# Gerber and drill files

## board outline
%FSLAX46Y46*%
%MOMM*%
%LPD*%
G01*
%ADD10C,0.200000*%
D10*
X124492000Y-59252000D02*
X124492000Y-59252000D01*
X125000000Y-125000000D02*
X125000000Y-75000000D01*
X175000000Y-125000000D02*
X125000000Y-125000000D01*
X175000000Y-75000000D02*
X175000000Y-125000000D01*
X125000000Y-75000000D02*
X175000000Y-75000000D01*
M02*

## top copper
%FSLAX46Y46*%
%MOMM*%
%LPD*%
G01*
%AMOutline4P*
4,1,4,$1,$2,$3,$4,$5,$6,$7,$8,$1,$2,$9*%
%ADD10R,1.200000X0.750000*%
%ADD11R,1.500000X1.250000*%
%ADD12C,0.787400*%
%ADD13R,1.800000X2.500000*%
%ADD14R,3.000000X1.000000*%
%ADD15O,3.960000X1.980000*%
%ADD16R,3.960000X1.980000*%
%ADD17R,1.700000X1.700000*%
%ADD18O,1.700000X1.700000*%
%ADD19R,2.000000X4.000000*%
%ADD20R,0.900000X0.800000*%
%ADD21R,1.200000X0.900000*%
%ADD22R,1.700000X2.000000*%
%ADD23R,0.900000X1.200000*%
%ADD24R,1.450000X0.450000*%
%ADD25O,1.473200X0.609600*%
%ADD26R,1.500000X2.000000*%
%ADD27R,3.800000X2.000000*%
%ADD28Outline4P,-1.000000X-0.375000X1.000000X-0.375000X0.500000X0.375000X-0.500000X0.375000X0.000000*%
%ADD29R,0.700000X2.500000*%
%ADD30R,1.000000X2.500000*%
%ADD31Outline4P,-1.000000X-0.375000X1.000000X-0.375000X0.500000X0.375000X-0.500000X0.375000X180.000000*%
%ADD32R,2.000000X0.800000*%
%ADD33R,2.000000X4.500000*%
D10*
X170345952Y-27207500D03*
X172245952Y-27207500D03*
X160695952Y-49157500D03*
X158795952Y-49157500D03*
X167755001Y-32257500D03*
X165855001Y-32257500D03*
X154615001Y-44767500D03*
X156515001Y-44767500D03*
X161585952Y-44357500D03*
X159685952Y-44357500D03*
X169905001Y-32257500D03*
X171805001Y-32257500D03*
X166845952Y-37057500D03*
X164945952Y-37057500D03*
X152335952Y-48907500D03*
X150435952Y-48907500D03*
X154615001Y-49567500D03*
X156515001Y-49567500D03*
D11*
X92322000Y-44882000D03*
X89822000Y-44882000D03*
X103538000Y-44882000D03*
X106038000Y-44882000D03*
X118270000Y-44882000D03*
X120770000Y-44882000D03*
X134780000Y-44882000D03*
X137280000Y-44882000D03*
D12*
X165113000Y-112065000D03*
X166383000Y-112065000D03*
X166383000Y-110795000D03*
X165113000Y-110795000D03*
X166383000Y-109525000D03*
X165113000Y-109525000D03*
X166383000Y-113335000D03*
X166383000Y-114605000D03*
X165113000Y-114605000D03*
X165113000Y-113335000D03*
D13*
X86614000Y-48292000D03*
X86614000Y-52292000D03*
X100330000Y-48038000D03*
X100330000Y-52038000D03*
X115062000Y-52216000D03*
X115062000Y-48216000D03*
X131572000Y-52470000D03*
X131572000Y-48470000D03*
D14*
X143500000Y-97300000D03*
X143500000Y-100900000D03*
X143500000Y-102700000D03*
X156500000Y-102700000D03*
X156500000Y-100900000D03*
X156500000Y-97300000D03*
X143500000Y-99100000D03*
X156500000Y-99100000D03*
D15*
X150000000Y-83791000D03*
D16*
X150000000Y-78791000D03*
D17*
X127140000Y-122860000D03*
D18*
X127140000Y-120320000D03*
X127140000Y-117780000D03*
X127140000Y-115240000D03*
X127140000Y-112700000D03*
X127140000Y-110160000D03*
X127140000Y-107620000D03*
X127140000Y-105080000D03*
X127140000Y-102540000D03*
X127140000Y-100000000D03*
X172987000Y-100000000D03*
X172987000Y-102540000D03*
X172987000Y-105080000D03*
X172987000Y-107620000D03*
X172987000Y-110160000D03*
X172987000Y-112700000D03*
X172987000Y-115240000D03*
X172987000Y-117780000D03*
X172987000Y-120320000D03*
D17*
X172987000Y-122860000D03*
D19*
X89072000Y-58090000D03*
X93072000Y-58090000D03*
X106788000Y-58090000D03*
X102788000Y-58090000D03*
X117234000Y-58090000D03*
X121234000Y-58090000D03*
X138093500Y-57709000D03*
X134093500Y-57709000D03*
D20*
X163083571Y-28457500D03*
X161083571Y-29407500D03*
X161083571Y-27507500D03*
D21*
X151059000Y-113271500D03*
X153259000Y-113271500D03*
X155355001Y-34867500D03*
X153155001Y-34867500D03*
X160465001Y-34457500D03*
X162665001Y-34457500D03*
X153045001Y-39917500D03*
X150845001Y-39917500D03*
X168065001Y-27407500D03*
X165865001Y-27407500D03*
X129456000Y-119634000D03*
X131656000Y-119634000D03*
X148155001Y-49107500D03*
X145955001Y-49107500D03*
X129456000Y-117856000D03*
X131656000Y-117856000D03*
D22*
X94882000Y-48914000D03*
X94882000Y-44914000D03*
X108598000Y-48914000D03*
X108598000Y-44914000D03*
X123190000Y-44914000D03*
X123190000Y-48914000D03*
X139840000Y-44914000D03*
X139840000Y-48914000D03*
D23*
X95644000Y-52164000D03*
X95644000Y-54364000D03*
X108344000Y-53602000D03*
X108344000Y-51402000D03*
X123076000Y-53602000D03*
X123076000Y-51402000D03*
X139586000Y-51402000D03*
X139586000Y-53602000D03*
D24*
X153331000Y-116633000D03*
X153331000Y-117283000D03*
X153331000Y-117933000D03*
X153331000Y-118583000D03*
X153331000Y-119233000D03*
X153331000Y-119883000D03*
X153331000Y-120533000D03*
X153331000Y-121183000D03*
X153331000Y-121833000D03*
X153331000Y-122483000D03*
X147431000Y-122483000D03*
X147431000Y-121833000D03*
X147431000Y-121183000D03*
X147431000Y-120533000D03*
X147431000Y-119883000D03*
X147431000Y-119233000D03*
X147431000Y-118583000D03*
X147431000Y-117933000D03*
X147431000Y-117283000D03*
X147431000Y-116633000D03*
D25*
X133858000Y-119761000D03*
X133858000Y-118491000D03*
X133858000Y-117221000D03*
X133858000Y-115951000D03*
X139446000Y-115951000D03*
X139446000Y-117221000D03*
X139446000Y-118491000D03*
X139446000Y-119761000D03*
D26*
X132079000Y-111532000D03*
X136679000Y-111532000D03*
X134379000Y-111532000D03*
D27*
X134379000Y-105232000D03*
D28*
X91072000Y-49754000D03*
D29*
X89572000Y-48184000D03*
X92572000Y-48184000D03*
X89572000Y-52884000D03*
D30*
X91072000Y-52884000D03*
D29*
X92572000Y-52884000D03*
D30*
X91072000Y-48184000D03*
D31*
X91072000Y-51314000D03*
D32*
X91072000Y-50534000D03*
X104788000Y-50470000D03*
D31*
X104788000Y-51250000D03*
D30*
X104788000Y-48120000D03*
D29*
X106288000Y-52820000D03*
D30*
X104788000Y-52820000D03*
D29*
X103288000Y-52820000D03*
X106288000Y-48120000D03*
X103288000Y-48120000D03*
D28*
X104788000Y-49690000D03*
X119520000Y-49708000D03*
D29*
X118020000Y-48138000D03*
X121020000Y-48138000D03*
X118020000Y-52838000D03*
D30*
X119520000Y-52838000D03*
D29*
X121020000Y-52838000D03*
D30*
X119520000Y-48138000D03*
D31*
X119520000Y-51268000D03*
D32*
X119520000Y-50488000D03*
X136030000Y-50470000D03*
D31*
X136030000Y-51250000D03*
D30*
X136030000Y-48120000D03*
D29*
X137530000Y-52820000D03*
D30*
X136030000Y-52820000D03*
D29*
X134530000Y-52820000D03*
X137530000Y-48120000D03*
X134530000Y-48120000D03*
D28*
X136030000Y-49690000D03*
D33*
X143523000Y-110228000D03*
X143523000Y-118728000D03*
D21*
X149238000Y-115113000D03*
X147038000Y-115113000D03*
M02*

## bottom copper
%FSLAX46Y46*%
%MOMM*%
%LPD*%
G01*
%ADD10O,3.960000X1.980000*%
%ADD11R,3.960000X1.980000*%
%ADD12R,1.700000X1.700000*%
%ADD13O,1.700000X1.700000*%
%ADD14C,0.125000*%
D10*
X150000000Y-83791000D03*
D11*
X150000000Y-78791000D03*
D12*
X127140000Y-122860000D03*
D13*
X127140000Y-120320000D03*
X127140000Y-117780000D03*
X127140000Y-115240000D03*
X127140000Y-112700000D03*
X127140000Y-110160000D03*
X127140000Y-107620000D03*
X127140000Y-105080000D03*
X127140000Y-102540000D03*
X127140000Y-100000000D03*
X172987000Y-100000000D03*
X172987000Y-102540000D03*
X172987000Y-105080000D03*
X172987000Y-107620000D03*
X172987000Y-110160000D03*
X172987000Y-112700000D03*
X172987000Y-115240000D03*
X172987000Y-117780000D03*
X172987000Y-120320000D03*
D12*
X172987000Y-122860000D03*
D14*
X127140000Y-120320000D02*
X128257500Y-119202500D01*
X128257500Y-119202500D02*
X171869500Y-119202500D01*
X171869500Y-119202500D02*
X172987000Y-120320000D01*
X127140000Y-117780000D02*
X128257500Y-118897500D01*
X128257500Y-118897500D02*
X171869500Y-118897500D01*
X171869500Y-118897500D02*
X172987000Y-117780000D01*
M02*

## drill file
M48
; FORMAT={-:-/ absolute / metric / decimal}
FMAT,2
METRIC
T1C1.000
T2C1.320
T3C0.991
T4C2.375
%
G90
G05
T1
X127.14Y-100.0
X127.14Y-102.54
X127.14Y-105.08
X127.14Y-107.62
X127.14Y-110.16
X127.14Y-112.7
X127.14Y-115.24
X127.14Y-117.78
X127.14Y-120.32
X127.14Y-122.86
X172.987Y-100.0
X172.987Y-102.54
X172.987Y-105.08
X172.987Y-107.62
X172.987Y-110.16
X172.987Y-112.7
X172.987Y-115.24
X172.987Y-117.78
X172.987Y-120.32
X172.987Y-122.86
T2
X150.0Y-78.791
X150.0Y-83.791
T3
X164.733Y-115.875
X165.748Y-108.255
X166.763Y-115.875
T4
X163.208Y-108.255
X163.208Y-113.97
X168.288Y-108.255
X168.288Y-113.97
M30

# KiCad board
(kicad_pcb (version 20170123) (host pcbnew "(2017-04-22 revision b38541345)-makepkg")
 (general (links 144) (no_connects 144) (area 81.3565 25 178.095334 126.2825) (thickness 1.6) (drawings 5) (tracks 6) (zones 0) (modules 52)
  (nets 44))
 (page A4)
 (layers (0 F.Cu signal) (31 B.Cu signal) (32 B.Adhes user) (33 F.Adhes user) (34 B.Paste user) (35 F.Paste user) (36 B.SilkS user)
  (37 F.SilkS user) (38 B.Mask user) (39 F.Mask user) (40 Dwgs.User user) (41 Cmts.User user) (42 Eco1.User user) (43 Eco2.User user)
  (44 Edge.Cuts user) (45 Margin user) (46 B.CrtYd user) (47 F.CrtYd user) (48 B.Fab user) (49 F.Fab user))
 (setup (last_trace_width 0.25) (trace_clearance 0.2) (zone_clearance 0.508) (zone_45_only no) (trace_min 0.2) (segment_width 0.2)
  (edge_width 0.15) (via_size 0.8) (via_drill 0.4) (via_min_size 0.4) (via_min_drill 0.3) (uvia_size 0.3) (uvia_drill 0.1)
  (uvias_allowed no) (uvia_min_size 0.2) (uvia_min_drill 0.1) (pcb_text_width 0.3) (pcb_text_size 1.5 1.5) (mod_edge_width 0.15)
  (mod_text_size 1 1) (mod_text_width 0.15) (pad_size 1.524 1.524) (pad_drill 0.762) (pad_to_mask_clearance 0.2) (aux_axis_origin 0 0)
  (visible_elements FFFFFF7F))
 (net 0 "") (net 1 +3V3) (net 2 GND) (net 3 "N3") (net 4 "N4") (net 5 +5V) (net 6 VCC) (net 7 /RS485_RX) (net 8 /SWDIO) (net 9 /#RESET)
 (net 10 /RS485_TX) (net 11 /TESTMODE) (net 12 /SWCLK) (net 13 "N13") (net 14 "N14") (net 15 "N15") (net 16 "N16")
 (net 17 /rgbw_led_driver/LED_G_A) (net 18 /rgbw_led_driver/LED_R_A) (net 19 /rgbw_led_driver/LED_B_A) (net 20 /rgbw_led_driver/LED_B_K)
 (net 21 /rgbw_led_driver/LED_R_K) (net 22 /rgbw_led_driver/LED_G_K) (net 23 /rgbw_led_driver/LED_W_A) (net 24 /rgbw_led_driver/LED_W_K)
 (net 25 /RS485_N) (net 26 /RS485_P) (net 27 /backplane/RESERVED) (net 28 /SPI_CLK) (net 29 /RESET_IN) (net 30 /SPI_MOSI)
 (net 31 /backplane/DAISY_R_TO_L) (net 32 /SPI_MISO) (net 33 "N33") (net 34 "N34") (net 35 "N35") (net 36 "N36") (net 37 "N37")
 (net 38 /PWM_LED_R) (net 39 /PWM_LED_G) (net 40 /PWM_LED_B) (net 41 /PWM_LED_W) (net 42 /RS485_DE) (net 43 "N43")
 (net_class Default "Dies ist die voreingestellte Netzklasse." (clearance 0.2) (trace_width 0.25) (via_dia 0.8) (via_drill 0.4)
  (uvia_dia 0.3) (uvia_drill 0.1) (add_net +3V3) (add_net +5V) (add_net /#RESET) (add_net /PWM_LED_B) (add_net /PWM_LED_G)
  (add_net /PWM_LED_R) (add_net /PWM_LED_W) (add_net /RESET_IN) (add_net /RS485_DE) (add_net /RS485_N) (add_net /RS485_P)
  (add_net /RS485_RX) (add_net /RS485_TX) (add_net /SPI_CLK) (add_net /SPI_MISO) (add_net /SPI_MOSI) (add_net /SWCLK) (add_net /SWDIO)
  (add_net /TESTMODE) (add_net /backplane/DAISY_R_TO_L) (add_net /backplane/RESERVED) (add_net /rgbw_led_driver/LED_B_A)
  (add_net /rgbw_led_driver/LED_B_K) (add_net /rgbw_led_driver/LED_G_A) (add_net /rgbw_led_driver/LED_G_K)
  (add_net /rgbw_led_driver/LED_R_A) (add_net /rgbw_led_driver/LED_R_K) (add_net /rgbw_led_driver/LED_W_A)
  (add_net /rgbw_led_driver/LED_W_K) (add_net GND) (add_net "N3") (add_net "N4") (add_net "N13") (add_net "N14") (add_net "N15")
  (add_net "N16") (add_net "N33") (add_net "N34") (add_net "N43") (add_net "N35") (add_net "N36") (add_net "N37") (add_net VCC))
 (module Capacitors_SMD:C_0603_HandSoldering (layer F.Cu) (at 171.295952 27.2075)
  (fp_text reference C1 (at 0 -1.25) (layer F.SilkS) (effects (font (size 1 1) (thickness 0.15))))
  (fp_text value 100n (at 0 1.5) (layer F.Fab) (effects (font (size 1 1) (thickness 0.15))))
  (pad 1 smd rect (at -0.95 0) (size 1.2 0.75) (layers F.Cu F.Paste F.Mask) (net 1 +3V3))
  (pad 2 smd rect (at 0.95 0) (size 1.2 0.75) (layers F.Cu F.Paste F.Mask) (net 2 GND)))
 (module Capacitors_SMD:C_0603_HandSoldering (layer F.Cu) (at 159.745952 49.1575)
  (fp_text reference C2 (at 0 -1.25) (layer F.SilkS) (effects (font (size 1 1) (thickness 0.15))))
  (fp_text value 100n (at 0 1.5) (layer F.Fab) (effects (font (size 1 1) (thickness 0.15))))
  (pad 2 smd rect (at 0.95 0) (size 1.2 0.75) (layers F.Cu F.Paste F.Mask) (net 2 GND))
  (pad 1 smd rect (at -0.95 0) (size 1.2 0.75) (layers F.Cu F.Paste F.Mask) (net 1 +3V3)))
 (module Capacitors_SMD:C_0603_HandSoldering (layer F.Cu) (at 166.805001 32.2575)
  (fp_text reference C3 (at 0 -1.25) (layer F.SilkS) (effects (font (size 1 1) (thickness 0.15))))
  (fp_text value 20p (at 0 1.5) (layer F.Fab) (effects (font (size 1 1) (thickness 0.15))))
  (pad 2 smd rect (at 0.95 0) (size 1.2 0.75) (layers F.Cu F.Paste F.Mask) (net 2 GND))
  (pad 1 smd rect (at -0.95 0) (size 1.2 0.75) (layers F.Cu F.Paste F.Mask) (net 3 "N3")))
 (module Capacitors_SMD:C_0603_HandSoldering (layer F.Cu) (at 155.565001 44.7675)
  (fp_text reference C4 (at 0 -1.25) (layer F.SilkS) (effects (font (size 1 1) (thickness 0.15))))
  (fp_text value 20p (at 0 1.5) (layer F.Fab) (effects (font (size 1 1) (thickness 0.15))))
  (pad 1 smd rect (at -0.95 0) (size 1.2 0.75) (layers F.Cu F.Paste F.Mask) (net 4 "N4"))
  (pad 2 smd rect (at 0.95 0) (size 1.2 0.75) (layers F.Cu F.Paste F.Mask) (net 2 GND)))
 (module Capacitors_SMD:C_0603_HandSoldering (layer F.Cu) (at 160.635952 44.3575)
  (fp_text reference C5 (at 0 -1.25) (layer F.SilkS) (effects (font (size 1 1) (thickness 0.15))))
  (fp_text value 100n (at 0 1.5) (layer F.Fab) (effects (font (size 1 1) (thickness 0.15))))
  (pad 2 smd rect (at 0.95 0) (size 1.2 0.75) (layers F.Cu F.Paste F.Mask) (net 2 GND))
  (pad 1 smd rect (at -0.95 0) (size 1.2 0.75) (layers F.Cu F.Paste F.Mask) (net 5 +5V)))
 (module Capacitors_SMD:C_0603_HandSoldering (layer F.Cu) (at 170.855001 32.2575)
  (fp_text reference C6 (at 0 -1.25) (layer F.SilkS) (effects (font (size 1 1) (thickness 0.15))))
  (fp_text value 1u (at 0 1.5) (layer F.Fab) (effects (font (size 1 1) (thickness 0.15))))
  (pad 1 smd rect (at -0.95 0) (size 1.2 0.75) (layers F.Cu F.Paste F.Mask) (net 5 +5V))
  (pad 2 smd rect (at 0.95 0) (size 1.2 0.75) (layers F.Cu F.Paste F.Mask) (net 2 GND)))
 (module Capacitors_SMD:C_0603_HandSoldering (layer F.Cu) (at 165.895952 37.0575)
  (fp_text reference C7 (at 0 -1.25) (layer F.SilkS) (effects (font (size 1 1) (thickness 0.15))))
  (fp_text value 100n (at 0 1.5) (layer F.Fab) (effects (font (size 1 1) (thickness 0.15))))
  (pad 2 smd rect (at 0.95 0) (size 1.2 0.75) (layers F.Cu F.Paste F.Mask) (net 2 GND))
  (pad 1 smd rect (at -0.95 0) (size 1.2 0.75) (layers F.Cu F.Paste F.Mask) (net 5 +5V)))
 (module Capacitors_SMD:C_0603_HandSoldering (layer F.Cu) (at 151.385952 48.9075)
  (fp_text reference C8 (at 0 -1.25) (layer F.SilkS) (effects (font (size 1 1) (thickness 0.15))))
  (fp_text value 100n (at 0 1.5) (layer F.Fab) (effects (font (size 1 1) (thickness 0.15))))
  (pad 2 smd rect (at 0.95 0) (size 1.2 0.75) (layers F.Cu F.Paste F.Mask) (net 2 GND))
  (pad 1 smd rect (at -0.95 0) (size 1.2 0.75) (layers F.Cu F.Paste F.Mask) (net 1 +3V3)))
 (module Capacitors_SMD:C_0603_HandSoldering (layer F.Cu) (at 155.565001 49.5675)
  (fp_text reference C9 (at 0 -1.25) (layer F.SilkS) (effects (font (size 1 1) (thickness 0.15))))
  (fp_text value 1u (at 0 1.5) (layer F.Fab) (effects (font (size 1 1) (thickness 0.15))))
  (pad 1 smd rect (at -0.95 0) (size 1.2 0.75) (layers F.Cu F.Paste F.Mask) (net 1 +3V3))
  (pad 2 smd rect (at 0.95 0) (size 1.2 0.75) (layers F.Cu F.Paste F.Mask) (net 2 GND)))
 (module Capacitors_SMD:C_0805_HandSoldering (layer F.Cu) (at 91.072 44.882)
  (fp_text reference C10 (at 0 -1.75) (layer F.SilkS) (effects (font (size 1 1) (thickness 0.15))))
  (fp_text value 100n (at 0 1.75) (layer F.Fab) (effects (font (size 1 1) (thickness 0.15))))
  (pad 2 smd rect (at 1.25 0) (size 1.5 1.25) (layers F.Cu F.Paste F.Mask) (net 2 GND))
  (pad 1 smd rect (at -1.25 0) (size 1.5 1.25) (layers F.Cu F.Paste F.Mask) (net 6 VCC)))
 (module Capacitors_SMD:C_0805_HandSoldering (layer F.Cu) (at 104.788 44.882)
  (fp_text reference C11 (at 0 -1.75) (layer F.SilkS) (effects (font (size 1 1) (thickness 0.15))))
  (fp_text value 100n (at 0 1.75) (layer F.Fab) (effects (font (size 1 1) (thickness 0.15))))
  (pad 1 smd rect (at -1.25 0) (size 1.5 1.25) (layers F.Cu F.Paste F.Mask) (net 6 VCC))
  (pad 2 smd rect (at 1.25 0) (size 1.5 1.25) (layers F.Cu F.Paste F.Mask) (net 2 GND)))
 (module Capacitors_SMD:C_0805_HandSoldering (layer F.Cu) (at 119.52 44.882)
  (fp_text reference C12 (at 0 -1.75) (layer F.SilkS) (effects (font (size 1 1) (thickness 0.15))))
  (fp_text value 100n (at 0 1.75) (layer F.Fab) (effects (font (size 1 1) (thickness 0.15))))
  (pad 1 smd rect (at -1.25 0) (size 1.5 1.25) (layers F.Cu F.Paste F.Mask) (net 6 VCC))
  (pad 2 smd rect (at 1.25 0) (size 1.5 1.25) (layers F.Cu F.Paste F.Mask) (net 2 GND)))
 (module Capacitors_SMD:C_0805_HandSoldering (layer F.Cu) (at 136.03 44.882)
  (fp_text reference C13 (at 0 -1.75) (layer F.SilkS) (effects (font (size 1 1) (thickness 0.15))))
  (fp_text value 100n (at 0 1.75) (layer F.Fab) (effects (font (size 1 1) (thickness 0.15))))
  (pad 1 smd rect (at -1.25 0) (size 1.5 1.25) (layers F.Cu F.Paste F.Mask) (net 6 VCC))
  (pad 2 smd rect (at 1.25 0) (size 1.5 1.25) (layers F.Cu F.Paste F.Mask) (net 2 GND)))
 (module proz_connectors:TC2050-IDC (layer F.Cu) (at 165.748 112.065 270)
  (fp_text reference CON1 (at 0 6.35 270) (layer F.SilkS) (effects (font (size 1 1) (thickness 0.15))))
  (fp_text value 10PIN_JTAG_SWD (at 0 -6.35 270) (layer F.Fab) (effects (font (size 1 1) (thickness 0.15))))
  (pad 3 smd circle (at 0 0.635 270) (size 0.7874 0.7874) (layers F.Cu F.Mask) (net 2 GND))
  (pad 8 smd circle (at 0 -0.635 270) (size 0.7874 0.7874) (layers F.Cu F.Mask))
  (pad 9 smd circle (at -1.27 -0.635 270) (size 0.7874 0.7874) (layers F.Cu F.Mask) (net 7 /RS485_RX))
  (pad 2 smd circle (at -1.27 0.635 270) (size 0.7874 0.7874) (layers F.Cu F.Mask) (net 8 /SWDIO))
  (pad 10 smd circle (at -2.54 -0.635 270) (size 0.7874 0.7874) (layers F.Cu F.Mask) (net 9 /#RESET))
  (pad 1 smd circle (at -2.54 0.635 270) (size 0.7874 0.7874) (layers F.Cu F.Mask) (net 1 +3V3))
  (pad 7 smd circle (at 1.27 -0.635 270) (size 0.7874 0.7874) (layers F.Cu F.Mask) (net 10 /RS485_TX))
  (pad 6 smd circle (at 2.54 -0.635 270) (size 0.7874 0.7874) (layers F.Cu F.Mask))
  (pad 5 smd circle (at 2.54 0.635 270) (size 0.7874 0.7874) (layers F.Cu F.Mask) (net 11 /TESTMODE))
  (pad 4 smd circle (at 1.27 0.635 270) (size 0.7874 0.7874) (layers F.Cu F.Mask) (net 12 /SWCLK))
  (pad "" np_thru_hole circle (at -3.81 -2.54 270) (size 2.375 2.375) (drill 2.375) (layers *.Cu *.Mask F.SilkS))
  (pad "" np_thru_hole circle (at -3.81 0 270) (size 0.9906 0.9906) (drill 0.9906) (layers *.Cu *.Mask F.SilkS))
  (pad "" np_thru_hole circle (at 3.81 -1.015 270) (size 0.9906 0.9906) (drill 0.9906) (layers *.Cu *.Mask F.SilkS))
  (pad "" np_thru_hole circle (at 3.81 1.015 270) (size 0.9906 0.9906) (drill 0.9906) (layers *.Cu *.Mask F.SilkS))
  (pad "" np_thru_hole circle (at -3.81 2.54 270) (size 2.375 2.375) (drill 2.375) (layers *.Cu *.Mask F.SilkS))
  (pad "" np_thru_hole circle (at 1.905 2.54 270) (size 2.375 2.375) (drill 2.375) (layers *.Cu *.Mask F.SilkS))
  (pad "" np_thru_hole circle (at 1.905 -2.54 270) (size 2.375 2.375) (drill 2.375) (layers *.Cu *.Mask F.SilkS)))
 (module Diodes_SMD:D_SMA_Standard (layer F.Cu) (at 86.614 50.292 270)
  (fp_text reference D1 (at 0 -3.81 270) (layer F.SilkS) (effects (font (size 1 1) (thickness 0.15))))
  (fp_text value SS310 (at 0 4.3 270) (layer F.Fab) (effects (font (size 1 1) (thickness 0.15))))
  (pad 1 smd rect (at -2 0 270) (size 2.5 1.8) (layers F.Cu F.Paste F.Mask) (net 6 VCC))
  (pad 2 smd rect (at 2 0 270) (size 2.5 1.8) (layers F.Cu F.Paste F.Mask) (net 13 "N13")))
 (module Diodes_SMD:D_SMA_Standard (layer F.Cu) (at 100.33 50.038 270)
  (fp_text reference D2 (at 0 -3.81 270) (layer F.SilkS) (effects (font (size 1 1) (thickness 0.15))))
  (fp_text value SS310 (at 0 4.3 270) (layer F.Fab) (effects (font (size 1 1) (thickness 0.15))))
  (pad 1 smd rect (at -2 0 270) (size 2.5 1.8) (layers F.Cu F.Paste F.Mask) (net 6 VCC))
  (pad 2 smd rect (at 2 0 270) (size 2.5 1.8) (layers F.Cu F.Paste F.Mask) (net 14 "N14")))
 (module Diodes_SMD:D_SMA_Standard (layer F.Cu) (at 115.062 50.216 270)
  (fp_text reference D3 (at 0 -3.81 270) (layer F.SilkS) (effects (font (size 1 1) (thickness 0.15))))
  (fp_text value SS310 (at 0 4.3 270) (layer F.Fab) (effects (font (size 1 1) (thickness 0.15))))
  (pad 2 smd rect (at 2 0 270) (size 2.5 1.8) (layers F.Cu F.Paste F.Mask) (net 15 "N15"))
  (pad 1 smd rect (at -2 0 270) (size 2.5 1.8) (layers F.Cu F.Paste F.Mask) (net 6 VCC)))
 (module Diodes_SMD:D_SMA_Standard (layer F.Cu) (at 131.572 50.47 270)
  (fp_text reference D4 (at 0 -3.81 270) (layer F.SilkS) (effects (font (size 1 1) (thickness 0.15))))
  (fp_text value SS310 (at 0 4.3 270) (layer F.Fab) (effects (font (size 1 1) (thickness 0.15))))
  (pad 2 smd rect (at 2 0 270) (size 2.5 1.8) (layers F.Cu F.Paste F.Mask) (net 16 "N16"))
  (pad 1 smd rect (at -2 0 270) (size 2.5 1.8) (layers F.Cu F.Paste F.Mask) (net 6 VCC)))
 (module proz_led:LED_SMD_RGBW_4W (layer F.Cu) (at 150 100)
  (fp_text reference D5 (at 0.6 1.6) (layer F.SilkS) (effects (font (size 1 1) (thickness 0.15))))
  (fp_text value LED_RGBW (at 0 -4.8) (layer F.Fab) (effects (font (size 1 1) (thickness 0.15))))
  (pad 8 smd rect (at -6.5 -2.7) (size 3 1) (layers F.Cu F.Paste F.Mask) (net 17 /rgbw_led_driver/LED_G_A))
  (pad 6 smd rect (at -6.5 0.9) (size 3 1) (layers F.Cu F.Paste F.Mask) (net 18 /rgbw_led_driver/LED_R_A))
  (pad 5 smd rect (at -6.5 2.7) (size 3 1) (layers F.Cu F.Paste F.Mask) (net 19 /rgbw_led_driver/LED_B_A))
  (pad 4 smd rect (at 6.5 2.7) (size 3 1) (layers F.Cu F.Paste F.Mask) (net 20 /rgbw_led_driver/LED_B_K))
  (pad 3 smd rect (at 6.5 0.9) (size 3 1) (layers F.Cu F.Paste F.Mask) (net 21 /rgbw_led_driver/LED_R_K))
  (pad 1 smd rect (at 6.5 -2.7) (size 3 1) (layers F.Cu F.Paste F.Mask) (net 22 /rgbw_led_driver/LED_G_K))
  (pad "" smd circle (at 0 0) (size 7.5 7.5) (layers F.Mask))
  (pad 7 smd rect (at -6.5 -0.9) (size 3 1) (layers F.Cu F.Paste F.Mask) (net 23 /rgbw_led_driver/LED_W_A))
  (pad 2 smd rect (at 6.5 -0.9) (size 3 1) (layers F.Cu F.Paste F.Mask) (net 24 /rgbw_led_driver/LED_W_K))
  (pad "" smd circle (at 0 0) (size 9 9) (layers B.Mask)))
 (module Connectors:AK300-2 (layer B.Cu) (at 150 78.791 270)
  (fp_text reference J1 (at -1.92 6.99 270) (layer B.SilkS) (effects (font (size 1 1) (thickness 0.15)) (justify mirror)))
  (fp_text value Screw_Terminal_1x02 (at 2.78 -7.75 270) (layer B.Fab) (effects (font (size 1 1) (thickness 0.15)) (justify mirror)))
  (pad 2 thru_hole oval (at 5 0 270) (size 1.98 3.96) (drill 1.32) (layers *.Cu B.Paste B.Mask) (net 2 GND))
  (pad 1 thru_hole rect (at 0 0 270) (size 1.98 3.96) (drill 1.32) (layers *.Cu B.Paste B.Mask) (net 6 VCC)))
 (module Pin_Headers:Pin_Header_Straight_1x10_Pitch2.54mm (layer B.Cu) (at 127.14 122.86)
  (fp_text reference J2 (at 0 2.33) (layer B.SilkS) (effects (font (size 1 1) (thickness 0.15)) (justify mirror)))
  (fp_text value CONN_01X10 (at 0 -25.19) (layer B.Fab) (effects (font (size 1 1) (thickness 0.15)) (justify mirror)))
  (pad 1 thru_hole rect (at 0 0) (size 1.7 1.7) (drill 1) (layers *.Cu *.Mask) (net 2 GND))
  (pad 2 thru_hole oval (at 0 -2.54) (size 1.7 1.7) (drill 1) (layers *.Cu *.Mask) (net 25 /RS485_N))
  (pad 3 thru_hole oval (at 0 -5.08) (size 1.7 1.7) (drill 1) (layers *.Cu *.Mask) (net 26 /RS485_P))
  (pad 4 thru_hole oval (at 0 -7.62) (size 1.7 1.7) (drill 1) (layers *.Cu *.Mask) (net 2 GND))
  (pad 5 thru_hole oval (at 0 -10.16) (size 1.7 1.7) (drill 1) (layers *.Cu *.Mask) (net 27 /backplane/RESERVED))
  (pad 6 thru_hole oval (at 0 -12.7) (size 1.7 1.7) (drill 1) (layers *.Cu *.Mask) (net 5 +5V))
  (pad 7 thru_hole oval (at 0 -15.24) (size 1.7 1.7) (drill 1) (layers *.Cu *.Mask) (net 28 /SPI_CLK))
  (pad 8 thru_hole oval (at 0 -17.78) (size 1.7 1.7) (drill 1) (layers *.Cu *.Mask) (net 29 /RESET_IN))
  (pad 9 thru_hole oval (at 0 -20.32) (size 1.7 1.7) (drill 1) (layers *.Cu *.Mask) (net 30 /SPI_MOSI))
  (pad 10 thru_hole oval (at 0 -22.86) (size 1.7 1.7) (drill 1) (layers *.Cu *.Mask) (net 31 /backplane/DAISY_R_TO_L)))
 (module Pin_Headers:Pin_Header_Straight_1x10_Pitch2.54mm (layer B.Cu) (at 172.987 122.86)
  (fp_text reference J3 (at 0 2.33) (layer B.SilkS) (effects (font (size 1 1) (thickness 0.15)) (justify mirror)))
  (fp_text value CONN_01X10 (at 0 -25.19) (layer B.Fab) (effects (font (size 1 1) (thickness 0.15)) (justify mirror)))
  (pad 10 thru_hole oval (at 0 -22.86) (size 1.7 1.7) (drill 1) (layers *.Cu *.Mask) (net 31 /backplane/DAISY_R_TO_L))
  (pad 9 thru_hole oval (at 0 -20.32) (size 1.7 1.7) (drill 1) (layers *.Cu *.Mask) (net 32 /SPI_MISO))
  (pad 8 thru_hole oval (at 0 -17.78) (size 1.7 1.7) (drill 1) (layers *.Cu *.Mask) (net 29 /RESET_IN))
  (pad 7 thru_hole oval (at 0 -15.24) (size 1.7 1.7) (drill 1) (layers *.Cu *.Mask) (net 28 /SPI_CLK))
  (pad 6 thru_hole oval (at 0 -12.7) (size 1.7 1.7) (drill 1) (layers *.Cu *.Mask) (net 5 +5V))
  (pad 5 thru_hole oval (at 0 -10.16) (size 1.7 1.7) (drill 1) (layers *.Cu *.Mask) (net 27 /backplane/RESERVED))
  (pad 4 thru_hole oval (at 0 -7.62) (size 1.7 1.7) (drill 1) (layers *.Cu *.Mask) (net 2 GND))
  (pad 3 thru_hole oval (at 0 -5.08) (size 1.7 1.7) (drill 1) (layers *.Cu *.Mask) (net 26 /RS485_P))
  (pad 2 thru_hole oval (at 0 -2.54) (size 1.7 1.7) (drill 1) (layers *.Cu *.Mask) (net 25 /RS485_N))
  (pad 1 thru_hole rect (at 0 0) (size 1.7 1.7) (drill 1) (layers *.Cu *.Mask) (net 2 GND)))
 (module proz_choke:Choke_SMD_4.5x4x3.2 (layer F.Cu) (at 91.072 58.09 180)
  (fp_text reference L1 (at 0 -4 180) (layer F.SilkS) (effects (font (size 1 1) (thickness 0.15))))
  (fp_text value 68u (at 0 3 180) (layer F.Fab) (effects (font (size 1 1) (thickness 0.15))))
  (pad 2 smd rect (at 2 0 180) (size 2 4) (layers F.Cu F.Paste F.Mask) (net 13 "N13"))
  (pad 1 smd rect (at -2 0 180) (size 2 4) (layers F.Cu F.Paste F.Mask) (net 21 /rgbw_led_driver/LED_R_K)))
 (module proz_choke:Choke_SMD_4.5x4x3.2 (layer F.Cu) (at 104.788 58.09 180)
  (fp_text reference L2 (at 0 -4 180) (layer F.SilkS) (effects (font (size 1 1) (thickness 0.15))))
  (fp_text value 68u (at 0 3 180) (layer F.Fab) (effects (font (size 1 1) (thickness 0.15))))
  (pad 1 smd rect (at -2 0 180) (size 2 4) (layers F.Cu F.Paste F.Mask) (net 22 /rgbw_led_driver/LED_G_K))
  (pad 2 smd rect (at 2 0 180) (size 2 4) (layers F.Cu F.Paste F.Mask) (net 14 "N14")))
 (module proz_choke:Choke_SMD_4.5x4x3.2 (layer F.Cu) (at 119.234 58.09 180)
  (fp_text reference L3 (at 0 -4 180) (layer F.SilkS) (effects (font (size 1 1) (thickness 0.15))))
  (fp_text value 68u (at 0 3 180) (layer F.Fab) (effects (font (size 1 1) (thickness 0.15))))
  (pad 2 smd rect (at 2 0 180) (size 2 4) (layers F.Cu F.Paste F.Mask) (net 15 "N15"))
  (pad 1 smd rect (at -2 0 180) (size 2 4) (layers F.Cu F.Paste F.Mask) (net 20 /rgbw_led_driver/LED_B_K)))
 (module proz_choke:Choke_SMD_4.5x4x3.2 (layer F.Cu) (at 136.0935 57.709 180)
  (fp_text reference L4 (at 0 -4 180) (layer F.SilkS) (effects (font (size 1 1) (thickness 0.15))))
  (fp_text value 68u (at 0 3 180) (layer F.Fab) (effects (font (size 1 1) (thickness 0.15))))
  (pad 1 smd rect (at -2 0 180) (size 2 4) (layers F.Cu F.Paste F.Mask) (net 24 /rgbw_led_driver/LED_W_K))
  (pad 2 smd rect (at 2 0 180) (size 2 4) (layers F.Cu F.Paste F.Mask) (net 16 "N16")))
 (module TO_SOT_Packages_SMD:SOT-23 (layer F.Cu) (at 162.083571 28.4575)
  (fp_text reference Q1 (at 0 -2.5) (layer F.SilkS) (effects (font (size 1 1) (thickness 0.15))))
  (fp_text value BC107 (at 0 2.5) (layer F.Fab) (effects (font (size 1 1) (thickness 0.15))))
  (pad 3 smd rect (at 1 0) (size 0.9 0.8) (layers F.Cu F.Paste F.Mask) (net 9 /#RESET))
  (pad 2 smd rect (at -1 0.95) (size 0.9 0.8) (layers F.Cu F.Paste F.Mask) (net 2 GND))
  (pad 1 smd rect (at -1 -0.95) (size 0.9 0.8) (layers F.Cu F.Paste F.Mask) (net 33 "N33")))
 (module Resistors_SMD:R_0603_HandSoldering (layer F.Cu) (at 152.159 113.2715)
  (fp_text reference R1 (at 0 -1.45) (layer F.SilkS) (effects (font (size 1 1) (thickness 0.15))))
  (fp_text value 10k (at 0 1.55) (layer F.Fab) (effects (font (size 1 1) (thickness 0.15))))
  (pad 1 smd rect (at -1.1 0) (size 1.2 0.9) (layers F.Cu F.Paste F.Mask) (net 2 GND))
  (pad 2 smd rect (at 1.1 0) (size 1.2 0.9) (layers F.Cu F.Paste F.Mask) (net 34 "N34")))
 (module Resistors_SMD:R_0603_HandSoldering (layer F.Cu) (at 154.255001 34.8675)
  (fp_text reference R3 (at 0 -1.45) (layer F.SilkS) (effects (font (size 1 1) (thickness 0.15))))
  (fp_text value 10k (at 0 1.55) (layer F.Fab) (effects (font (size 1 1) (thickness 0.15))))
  (pad 2 smd rect (at 1.1 0) (size 1.2 0.9) (layers F.Cu F.Paste F.Mask) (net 1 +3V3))
  (pad 1 smd rect (at -1.1 0) (size 1.2 0.9) (layers F.Cu F.Paste F.Mask) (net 9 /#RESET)))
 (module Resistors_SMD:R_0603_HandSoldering (layer F.Cu) (at 161.565001 34.4575)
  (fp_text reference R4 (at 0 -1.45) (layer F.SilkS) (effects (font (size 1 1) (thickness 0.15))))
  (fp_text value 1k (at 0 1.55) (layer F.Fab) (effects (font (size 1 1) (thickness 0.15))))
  (pad 1 smd rect (at -1.1 0) (size 1.2 0.9) (layers F.Cu F.Paste F.Mask) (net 33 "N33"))
  (pad 2 smd rect (at 1.1 0) (size 1.2 0.9) (layers F.Cu F.Paste F.Mask) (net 29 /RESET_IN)))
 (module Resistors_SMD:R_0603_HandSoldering (layer F.Cu) (at 151.945001 39.9175)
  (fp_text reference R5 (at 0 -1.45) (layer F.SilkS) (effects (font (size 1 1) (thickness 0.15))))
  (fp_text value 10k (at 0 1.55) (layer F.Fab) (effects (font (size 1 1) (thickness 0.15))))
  (pad 2 smd rect (at 1.1 0) (size 1.2 0.9) (layers F.Cu F.Paste F.Mask) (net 33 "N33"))
  (pad 1 smd rect (at -1.1 0) (size 1.2 0.9) (layers F.Cu F.Paste F.Mask) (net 2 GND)))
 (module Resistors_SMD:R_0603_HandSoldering (layer F.Cu) (at 166.965001 27.4075)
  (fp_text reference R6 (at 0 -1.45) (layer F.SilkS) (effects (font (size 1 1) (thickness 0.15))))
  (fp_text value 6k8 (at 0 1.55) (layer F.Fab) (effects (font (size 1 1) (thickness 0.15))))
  (pad 2 smd rect (at 1.1 0) (size 1.2 0.9) (layers F.Cu F.Paste F.Mask) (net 7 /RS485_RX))
  (pad 1 smd rect (at -1.1 0) (size 1.2 0.9) (layers F.Cu F.Paste F.Mask) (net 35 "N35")))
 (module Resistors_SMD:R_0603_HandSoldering (layer F.Cu) (at 130.556 119.634)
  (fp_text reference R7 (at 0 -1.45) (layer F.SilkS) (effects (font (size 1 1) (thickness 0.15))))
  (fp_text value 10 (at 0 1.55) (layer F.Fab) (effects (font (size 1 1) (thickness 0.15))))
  (pad 1 smd rect (at -1.1 0) (size 1.2 0.9) (layers F.Cu F.Paste F.Mask) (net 25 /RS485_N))
  (pad 2 smd rect (at 1.1 0) (size 1.2 0.9) (layers F.Cu F.Paste F.Mask) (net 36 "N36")))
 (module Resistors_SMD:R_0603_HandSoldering (layer F.Cu) (at 147.055001 49.1075)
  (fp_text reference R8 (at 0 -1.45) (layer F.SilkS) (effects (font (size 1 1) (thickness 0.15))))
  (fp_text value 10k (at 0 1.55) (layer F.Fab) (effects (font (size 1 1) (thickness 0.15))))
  (pad 2 smd rect (at 1.1 0) (size 1.2 0.9) (layers F.Cu F.Paste F.Mask) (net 7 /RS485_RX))
  (pad 1 smd rect (at -1.1 0) (size 1.2 0.9) (layers F.Cu F.Paste F.Mask) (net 2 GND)))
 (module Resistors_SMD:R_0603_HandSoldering (layer F.Cu) (at 130.556 117.856)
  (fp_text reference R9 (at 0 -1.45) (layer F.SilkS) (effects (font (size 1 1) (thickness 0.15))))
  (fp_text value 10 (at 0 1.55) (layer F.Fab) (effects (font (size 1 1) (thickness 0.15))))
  (pad 1 smd rect (at -1.1 0) (size 1.2 0.9) (layers F.Cu F.Paste F.Mask) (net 26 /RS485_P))
  (pad 2 smd rect (at 1.1 0) (size 1.2 0.9) (layers F.Cu F.Paste F.Mask) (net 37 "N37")))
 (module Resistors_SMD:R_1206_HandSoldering (layer F.Cu) (at 94.882 46.914 90)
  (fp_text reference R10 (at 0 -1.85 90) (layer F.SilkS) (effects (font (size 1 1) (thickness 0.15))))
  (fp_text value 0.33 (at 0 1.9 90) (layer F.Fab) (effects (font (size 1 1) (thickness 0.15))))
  (pad 1 smd rect (at -2 0 90) (size 2 1.7) (layers F.Cu F.Paste F.Mask) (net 18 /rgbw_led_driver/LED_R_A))
  (pad 2 smd rect (at 2 0 90) (size 2 1.7) (layers F.Cu F.Paste F.Mask) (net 6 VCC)))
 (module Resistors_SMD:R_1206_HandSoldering (layer F.Cu) (at 108.598 46.914 90)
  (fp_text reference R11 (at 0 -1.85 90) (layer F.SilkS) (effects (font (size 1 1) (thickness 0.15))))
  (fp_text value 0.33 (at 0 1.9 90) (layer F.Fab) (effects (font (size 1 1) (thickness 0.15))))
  (pad 1 smd rect (at -2 0 90) (size 2 1.7) (layers F.Cu F.Paste F.Mask) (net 17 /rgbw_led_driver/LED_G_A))
  (pad 2 smd rect (at 2 0 90) (size 2 1.7) (layers F.Cu F.Paste F.Mask) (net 6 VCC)))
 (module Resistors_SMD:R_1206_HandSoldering (layer F.Cu) (at 123.19 46.914 90)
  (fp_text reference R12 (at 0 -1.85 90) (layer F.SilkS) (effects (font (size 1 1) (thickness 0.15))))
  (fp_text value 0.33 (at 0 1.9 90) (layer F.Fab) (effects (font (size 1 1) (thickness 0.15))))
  (pad 2 smd rect (at 2 0 90) (size 2 1.7) (layers F.Cu F.Paste F.Mask) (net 6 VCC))
  (pad 1 smd rect (at -2 0 90) (size 2 1.7) (layers F.Cu F.Paste F.Mask) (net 19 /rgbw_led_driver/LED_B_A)))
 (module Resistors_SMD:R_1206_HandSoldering (layer F.Cu) (at 139.84 46.914 90)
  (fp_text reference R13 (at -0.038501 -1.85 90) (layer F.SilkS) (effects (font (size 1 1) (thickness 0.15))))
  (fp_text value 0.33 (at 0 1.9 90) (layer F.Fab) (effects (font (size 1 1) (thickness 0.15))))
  (pad 2 smd rect (at 2 0 90) (size 2 1.7) (layers F.Cu F.Paste F.Mask) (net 6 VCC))
  (pad 1 smd rect (at -2 0 90) (size 2 1.7) (layers F.Cu F.Paste F.Mask) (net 23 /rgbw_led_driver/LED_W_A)))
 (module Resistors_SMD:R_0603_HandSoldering (layer F.Cu) (at 95.644 53.264 90)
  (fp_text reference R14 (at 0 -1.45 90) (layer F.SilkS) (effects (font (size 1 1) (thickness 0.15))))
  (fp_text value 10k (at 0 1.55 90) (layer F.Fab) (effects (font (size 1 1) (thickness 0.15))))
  (pad 2 smd rect (at 1.1 0 90) (size 1.2 0.9) (layers F.Cu F.Paste F.Mask) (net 2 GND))
  (pad 1 smd rect (at -1.1 0 90) (size 1.2 0.9) (layers F.Cu F.Paste F.Mask) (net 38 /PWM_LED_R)))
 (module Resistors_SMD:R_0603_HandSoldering (layer F.Cu) (at 108.344 52.502 90)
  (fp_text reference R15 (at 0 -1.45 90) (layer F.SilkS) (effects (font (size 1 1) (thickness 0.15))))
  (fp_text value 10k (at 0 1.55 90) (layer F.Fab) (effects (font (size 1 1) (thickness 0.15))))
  (pad 1 smd rect (at -1.1 0 90) (size 1.2 0.9) (layers F.Cu F.Paste F.Mask) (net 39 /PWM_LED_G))
  (pad 2 smd rect (at 1.1 0 90) (size 1.2 0.9) (layers F.Cu F.Paste F.Mask) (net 2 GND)))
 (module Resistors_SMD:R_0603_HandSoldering (layer F.Cu) (at 123.076 52.502 90)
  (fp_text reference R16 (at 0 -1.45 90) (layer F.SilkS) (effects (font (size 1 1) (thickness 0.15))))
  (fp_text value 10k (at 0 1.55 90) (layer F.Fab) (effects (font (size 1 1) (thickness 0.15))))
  (pad 1 smd rect (at -1.1 0 90) (size 1.2 0.9) (layers F.Cu F.Paste F.Mask) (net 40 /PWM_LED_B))
  (pad 2 smd rect (at 1.1 0 90) (size 1.2 0.9) (layers F.Cu F.Paste F.Mask) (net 2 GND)))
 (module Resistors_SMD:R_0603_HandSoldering (layer F.Cu) (at 139.586 52.502 90)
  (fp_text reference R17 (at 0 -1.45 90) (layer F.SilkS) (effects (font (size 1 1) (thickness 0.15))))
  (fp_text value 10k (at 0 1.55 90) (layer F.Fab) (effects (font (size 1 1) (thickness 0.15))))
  (pad 2 smd rect (at 1.1 0 90) (size 1.2 0.9) (layers F.Cu F.Paste F.Mask) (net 2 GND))
  (pad 1 smd rect (at -1.1 0 90) (size 1.2 0.9) (layers F.Cu F.Paste F.Mask) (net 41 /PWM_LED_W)))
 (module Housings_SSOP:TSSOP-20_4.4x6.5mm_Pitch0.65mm (layer F.Cu) (at 150.381 119.558)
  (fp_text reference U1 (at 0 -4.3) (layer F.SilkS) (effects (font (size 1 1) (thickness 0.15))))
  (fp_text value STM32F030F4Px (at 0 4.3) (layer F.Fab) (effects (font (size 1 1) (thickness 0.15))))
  (pad 20 smd rect (at 2.95 -2.925) (size 1.45 0.45) (layers F.Cu F.Paste F.Mask) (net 12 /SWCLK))
  (pad 19 smd rect (at 2.95 -2.275) (size 1.45 0.45) (layers F.Cu F.Paste F.Mask) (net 8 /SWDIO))
  (pad 18 smd rect (at 2.95 -1.625) (size 1.45 0.45) (layers F.Cu F.Paste F.Mask) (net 40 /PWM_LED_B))
  (pad 17 smd rect (at 2.95 -0.975) (size 1.45 0.45) (layers F.Cu F.Paste F.Mask) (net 39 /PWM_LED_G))
  (pad 16 smd rect (at 2.95 -0.325) (size 1.45 0.45) (layers F.Cu F.Paste F.Mask) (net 1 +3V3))
  (pad 15 smd rect (at 2.95 0.325) (size 1.45 0.45) (layers F.Cu F.Paste F.Mask) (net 2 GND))
  (pad 14 smd rect (at 2.95 0.975) (size 1.45 0.45) (layers F.Cu F.Paste F.Mask) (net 41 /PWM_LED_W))
  (pad 13 smd rect (at 2.95 1.625) (size 1.45 0.45) (layers F.Cu F.Paste F.Mask) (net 30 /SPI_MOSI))
  (pad 12 smd rect (at 2.95 2.275) (size 1.45 0.45) (layers F.Cu F.Paste F.Mask) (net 32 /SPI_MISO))
  (pad 11 smd rect (at 2.95 2.925) (size 1.45 0.45) (layers F.Cu F.Paste F.Mask) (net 28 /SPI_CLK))
  (pad 10 smd rect (at -2.95 2.925) (size 1.45 0.45) (layers F.Cu F.Paste F.Mask) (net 38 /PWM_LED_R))
  (pad 9 smd rect (at -2.95 2.275) (size 1.45 0.45) (layers F.Cu F.Paste F.Mask) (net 7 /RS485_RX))
  (pad 8 smd rect (at -2.95 1.625) (size 1.45 0.45) (layers F.Cu F.Paste F.Mask) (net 10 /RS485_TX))
  (pad 7 smd rect (at -2.95 0.975) (size 1.45 0.45) (layers F.Cu F.Paste F.Mask) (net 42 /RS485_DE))
  (pad 6 smd rect (at -2.95 0.325) (size 1.45 0.45) (layers F.Cu F.Paste F.Mask) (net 11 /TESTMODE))
  (pad 5 smd rect (at -2.95 -0.325) (size 1.45 0.45) (layers F.Cu F.Paste F.Mask) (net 1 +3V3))
  (pad 4 smd rect (at -2.95 -0.975) (size 1.45 0.45) (layers F.Cu F.Paste F.Mask) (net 9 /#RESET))
  (pad 3 smd rect (at -2.95 -1.625) (size 1.45 0.45) (layers F.Cu F.Paste F.Mask) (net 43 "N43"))
  (pad 2 smd rect (at -2.95 -2.275) (size 1.45 0.45) (layers F.Cu F.Paste F.Mask) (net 3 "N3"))
  (pad 1 smd rect (at -2.95 -2.925) (size 1.45 0.45) (layers F.Cu F.Paste F.Mask) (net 34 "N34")))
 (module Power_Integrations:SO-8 (layer F.Cu) (at 136.652 117.856 90)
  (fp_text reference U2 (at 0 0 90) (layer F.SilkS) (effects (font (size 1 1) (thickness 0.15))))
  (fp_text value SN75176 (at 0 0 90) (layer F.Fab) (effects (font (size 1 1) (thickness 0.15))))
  (pad 8 smd oval (at -1.905 -2.794 90) (size 0.6096 1.4732) (layers F.Cu F.Paste F.Mask) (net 5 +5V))
  (pad 7 smd oval (at -0.635 -2.794 90) (size 0.6096 1.4732) (layers F.Cu F.Paste F.Mask) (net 36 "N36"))
  (pad 6 smd oval (at 0.635 -2.794 90) (size 0.6096 1.4732) (layers F.Cu F.Paste F.Mask) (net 37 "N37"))
  (pad 5 smd oval (at 1.905 -2.794 90) (size 0.6096 1.4732) (layers F.Cu F.Paste F.Mask) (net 2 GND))
  (pad 4 smd oval (at 1.905 2.794 90) (size 0.6096 1.4732) (layers F.Cu F.Paste F.Mask) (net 10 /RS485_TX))
  (pad 3 smd oval (at 0.635 2.794 90) (size 0.6096 1.4732) (layers F.Cu F.Paste F.Mask) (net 42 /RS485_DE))
  (pad 2 smd oval (at -0.635 2.794 90) (size 0.6096 1.4732) (layers F.Cu F.Paste F.Mask) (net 42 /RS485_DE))
  (pad 1 smd oval (at -1.905 2.794 90) (size 0.6096 1.4732) (layers F.Cu F.Paste F.Mask) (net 35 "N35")))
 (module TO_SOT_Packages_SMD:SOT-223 (layer F.Cu) (at 134.379 108.382 90)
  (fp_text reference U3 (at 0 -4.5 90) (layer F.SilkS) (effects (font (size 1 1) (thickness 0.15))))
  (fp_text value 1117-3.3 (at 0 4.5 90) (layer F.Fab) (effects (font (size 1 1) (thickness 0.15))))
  (pad 1 smd rect (at -3.15 -2.3 90) (size 2 1.5) (layers F.Cu F.Paste F.Mask) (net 2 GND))
  (pad 3 smd rect (at -3.15 2.3 90) (size 2 1.5) (layers F.Cu F.Paste F.Mask) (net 5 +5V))
  (pad 2 smd rect (at -3.15 0 90) (size 2 1.5) (layers F.Cu F.Paste F.Mask) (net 1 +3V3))
  (pad 4 smd rect (at 3.15 0 90) (size 2 3.8) (layers F.Cu F.Paste F.Mask) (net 1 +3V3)))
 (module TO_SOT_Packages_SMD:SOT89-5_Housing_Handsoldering (layer F.Cu) (at 91.072 50.534 90)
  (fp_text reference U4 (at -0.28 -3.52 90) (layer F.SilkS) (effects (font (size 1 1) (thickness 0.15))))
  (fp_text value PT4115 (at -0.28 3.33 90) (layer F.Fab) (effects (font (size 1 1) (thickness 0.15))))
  (pad 2 smd trapezoid (at 0.78 0) (size 1.5 0.75) (rect_delta 0 0.5) (layers F.Cu F.Paste F.Mask) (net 2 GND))
  (pad 5 smd rect (at 2.35 -1.5) (size 0.7 2.5) (layers F.Cu F.Paste F.Mask) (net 6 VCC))
  (pad 4 smd rect (at 2.35 1.5) (size 0.7 2.5) (layers F.Cu F.Paste F.Mask) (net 18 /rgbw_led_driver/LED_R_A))
  (pad 1 smd rect (at -2.35 -1.5) (size 0.7 2.5) (layers F.Cu F.Paste F.Mask) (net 13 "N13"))
  (pad 2 smd rect (at -2.35 0) (size 1 2.5) (layers F.Cu F.Paste F.Mask) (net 2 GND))
  (pad 3 smd rect (at -2.35 1.5) (size 0.7 2.5) (layers F.Cu F.Paste F.Mask) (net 38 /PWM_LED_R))
  (pad 2 smd rect (at 2.35 0) (size 1 2.5) (layers F.Cu F.Paste F.Mask) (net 2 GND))
  (pad 2 smd trapezoid (at -0.78 0 180) (size 1.5 0.75) (rect_delta 0 0.5) (layers F.Cu F.Paste F.Mask) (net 2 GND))
  (pad 2 smd rect (at 0 0) (size 2 0.8) (layers F.Cu F.Paste F.Mask) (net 2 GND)))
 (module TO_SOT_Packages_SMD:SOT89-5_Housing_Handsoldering (layer F.Cu) (at 104.788 50.47 90)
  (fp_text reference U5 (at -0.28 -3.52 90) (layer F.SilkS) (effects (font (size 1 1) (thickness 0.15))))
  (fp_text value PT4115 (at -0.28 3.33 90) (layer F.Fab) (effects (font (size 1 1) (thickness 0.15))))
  (pad 2 smd rect (at 0 0) (size 2 0.8) (layers F.Cu F.Paste F.Mask) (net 2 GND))
  (pad 2 smd trapezoid (at -0.78 0 180) (size 1.5 0.75) (rect_delta 0 0.5) (layers F.Cu F.Paste F.Mask) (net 2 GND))
  (pad 2 smd rect (at 2.35 0) (size 1 2.5) (layers F.Cu F.Paste F.Mask) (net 2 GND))
  (pad 3 smd rect (at -2.35 1.5) (size 0.7 2.5) (layers F.Cu F.Paste F.Mask) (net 39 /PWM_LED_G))
  (pad 2 smd rect (at -2.35 0) (size 1 2.5) (layers F.Cu F.Paste F.Mask) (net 2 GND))
  (pad 1 smd rect (at -2.35 -1.5) (size 0.7 2.5) (layers F.Cu F.Paste F.Mask) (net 14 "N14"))
  (pad 4 smd rect (at 2.35 1.5) (size 0.7 2.5) (layers F.Cu F.Paste F.Mask) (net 17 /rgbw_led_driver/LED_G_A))
  (pad 5 smd rect (at 2.35 -1.5) (size 0.7 2.5) (layers F.Cu F.Paste F.Mask) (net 6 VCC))
  (pad 2 smd trapezoid (at 0.78 0) (size 1.5 0.75) (rect_delta 0 0.5) (layers F.Cu F.Paste F.Mask) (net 2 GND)))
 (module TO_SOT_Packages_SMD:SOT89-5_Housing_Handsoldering (layer F.Cu) (at 119.52 50.488 90)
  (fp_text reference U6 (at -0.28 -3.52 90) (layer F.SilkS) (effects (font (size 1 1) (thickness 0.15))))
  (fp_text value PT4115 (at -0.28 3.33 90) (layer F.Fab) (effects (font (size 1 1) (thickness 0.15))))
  (pad 2 smd trapezoid (at 0.78 0) (size 1.5 0.75) (rect_delta 0 0.5) (layers F.Cu F.Paste F.Mask) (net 2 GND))
  (pad 5 smd rect (at 2.35 -1.5) (size 0.7 2.5) (layers F.Cu F.Paste F.Mask) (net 6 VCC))
  (pad 4 smd rect (at 2.35 1.5) (size 0.7 2.5) (layers F.Cu F.Paste F.Mask) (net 19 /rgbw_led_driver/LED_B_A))
  (pad 1 smd rect (at -2.35 -1.5) (size 0.7 2.5) (layers F.Cu F.Paste F.Mask) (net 15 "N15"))
  (pad 2 smd rect (at -2.35 0) (size 1 2.5) (layers F.Cu F.Paste F.Mask) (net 2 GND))
  (pad 3 smd rect (at -2.35 1.5) (size 0.7 2.5) (layers F.Cu F.Paste F.Mask) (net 40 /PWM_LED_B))
  (pad 2 smd rect (at 2.35 0) (size 1 2.5) (layers F.Cu F.Paste F.Mask) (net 2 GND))
  (pad 2 smd trapezoid (at -0.78 0 180) (size 1.5 0.75) (rect_delta 0 0.5) (layers F.Cu F.Paste F.Mask) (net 2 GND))
  (pad 2 smd rect (at 0 0) (size 2 0.8) (layers F.Cu F.Paste F.Mask) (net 2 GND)))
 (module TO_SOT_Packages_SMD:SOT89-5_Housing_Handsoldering (layer F.Cu) (at 136.03 50.47 90)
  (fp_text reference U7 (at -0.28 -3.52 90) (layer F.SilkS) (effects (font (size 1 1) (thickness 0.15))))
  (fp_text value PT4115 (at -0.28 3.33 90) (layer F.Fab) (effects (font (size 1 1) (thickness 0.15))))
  (pad 2 smd rect (at 0 0) (size 2 0.8) (layers F.Cu F.Paste F.Mask) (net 2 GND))
  (pad 2 smd trapezoid (at -0.78 0 180) (size 1.5 0.75) (rect_delta 0 0.5) (layers F.Cu F.Paste F.Mask) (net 2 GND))
  (pad 2 smd rect (at 2.35 0) (size 1 2.5) (layers F.Cu F.Paste F.Mask) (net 2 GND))
  (pad 3 smd rect (at -2.35 1.5) (size 0.7 2.5) (layers F.Cu F.Paste F.Mask) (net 41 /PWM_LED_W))
  (pad 2 smd rect (at -2.35 0) (size 1 2.5) (layers F.Cu F.Paste F.Mask) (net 2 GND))
  (pad 1 smd rect (at -2.35 -1.5) (size 0.7 2.5) (layers F.Cu F.Paste F.Mask) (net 16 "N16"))
  (pad 4 smd rect (at 2.35 1.5) (size 0.7 2.5) (layers F.Cu F.Paste F.Mask) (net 23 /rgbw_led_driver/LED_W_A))
  (pad 5 smd rect (at 2.35 -1.5) (size 0.7 2.5) (layers F.Cu F.Paste F.Mask) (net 6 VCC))
  (pad 2 smd trapezoid (at 0.78 0) (size 1.5 0.75) (rect_delta 0 0.5) (layers F.Cu F.Paste F.Mask) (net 2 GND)))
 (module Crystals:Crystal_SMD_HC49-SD (layer F.Cu) (at 143.523 114.478 90)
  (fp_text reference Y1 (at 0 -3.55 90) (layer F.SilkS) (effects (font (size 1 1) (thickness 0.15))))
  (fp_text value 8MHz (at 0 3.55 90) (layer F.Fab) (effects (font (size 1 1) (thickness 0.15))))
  (pad 2 smd rect (at 4.25 0 90) (size 4.5 2) (layers F.Cu F.Paste F.Mask) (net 4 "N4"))
  (pad 1 smd rect (at -4.25 0 90) (size 4.5 2) (layers F.Cu F.Paste F.Mask) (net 3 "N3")))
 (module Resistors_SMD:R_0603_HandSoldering (layer F.Cu) (at 148.138 115.113)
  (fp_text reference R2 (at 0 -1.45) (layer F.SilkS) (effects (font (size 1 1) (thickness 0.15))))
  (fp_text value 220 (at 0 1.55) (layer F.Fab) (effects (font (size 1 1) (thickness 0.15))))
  (pad 2 smd rect (at 1.1 0) (size 1.2 0.9) (layers F.Cu F.Paste F.Mask) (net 43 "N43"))
  (pad 1 smd rect (at -1.1 0) (size 1.2 0.9) (layers F.Cu F.Paste F.Mask) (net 4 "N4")))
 (gr_line (start 124.492 59.252) (end 124.492 59.252) (layer Edge.Cuts) (width 0.2))
 (gr_line (start 125 125) (end 125 75) (layer Edge.Cuts) (width 0.2))
 (gr_line (start 175 125) (end 125 125) (layer Edge.Cuts) (width 0.2))
 (gr_line (start 175 75) (end 175 125) (layer Edge.Cuts) (width 0.2))
 (gr_line (start 125 75) (end 175 75) (layer Edge.Cuts) (width 0.2))
 (segment (start 127.14 120.32) (end 128.2575 119.2025) (width 0.125) (layer B.Cu) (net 25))
 (segment (start 128.2575 119.2025) (end 171.8695 119.2025) (width 0.125) (layer B.Cu) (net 25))
 (segment (start 171.8695 119.2025) (end 172.987 120.32) (width 0.125) (layer B.Cu) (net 25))
 (segment (start 127.14 117.78) (end 128.2575 118.8975) (width 0.125) (layer B.Cu) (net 26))
 (segment (start 128.2575 118.8975) (end 171.8695 118.8975) (width 0.125) (layer B.Cu) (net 26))
 (segment (start 171.8695 118.8975) (end 172.987 117.78) (width 0.125) (layer B.Cu) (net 26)))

